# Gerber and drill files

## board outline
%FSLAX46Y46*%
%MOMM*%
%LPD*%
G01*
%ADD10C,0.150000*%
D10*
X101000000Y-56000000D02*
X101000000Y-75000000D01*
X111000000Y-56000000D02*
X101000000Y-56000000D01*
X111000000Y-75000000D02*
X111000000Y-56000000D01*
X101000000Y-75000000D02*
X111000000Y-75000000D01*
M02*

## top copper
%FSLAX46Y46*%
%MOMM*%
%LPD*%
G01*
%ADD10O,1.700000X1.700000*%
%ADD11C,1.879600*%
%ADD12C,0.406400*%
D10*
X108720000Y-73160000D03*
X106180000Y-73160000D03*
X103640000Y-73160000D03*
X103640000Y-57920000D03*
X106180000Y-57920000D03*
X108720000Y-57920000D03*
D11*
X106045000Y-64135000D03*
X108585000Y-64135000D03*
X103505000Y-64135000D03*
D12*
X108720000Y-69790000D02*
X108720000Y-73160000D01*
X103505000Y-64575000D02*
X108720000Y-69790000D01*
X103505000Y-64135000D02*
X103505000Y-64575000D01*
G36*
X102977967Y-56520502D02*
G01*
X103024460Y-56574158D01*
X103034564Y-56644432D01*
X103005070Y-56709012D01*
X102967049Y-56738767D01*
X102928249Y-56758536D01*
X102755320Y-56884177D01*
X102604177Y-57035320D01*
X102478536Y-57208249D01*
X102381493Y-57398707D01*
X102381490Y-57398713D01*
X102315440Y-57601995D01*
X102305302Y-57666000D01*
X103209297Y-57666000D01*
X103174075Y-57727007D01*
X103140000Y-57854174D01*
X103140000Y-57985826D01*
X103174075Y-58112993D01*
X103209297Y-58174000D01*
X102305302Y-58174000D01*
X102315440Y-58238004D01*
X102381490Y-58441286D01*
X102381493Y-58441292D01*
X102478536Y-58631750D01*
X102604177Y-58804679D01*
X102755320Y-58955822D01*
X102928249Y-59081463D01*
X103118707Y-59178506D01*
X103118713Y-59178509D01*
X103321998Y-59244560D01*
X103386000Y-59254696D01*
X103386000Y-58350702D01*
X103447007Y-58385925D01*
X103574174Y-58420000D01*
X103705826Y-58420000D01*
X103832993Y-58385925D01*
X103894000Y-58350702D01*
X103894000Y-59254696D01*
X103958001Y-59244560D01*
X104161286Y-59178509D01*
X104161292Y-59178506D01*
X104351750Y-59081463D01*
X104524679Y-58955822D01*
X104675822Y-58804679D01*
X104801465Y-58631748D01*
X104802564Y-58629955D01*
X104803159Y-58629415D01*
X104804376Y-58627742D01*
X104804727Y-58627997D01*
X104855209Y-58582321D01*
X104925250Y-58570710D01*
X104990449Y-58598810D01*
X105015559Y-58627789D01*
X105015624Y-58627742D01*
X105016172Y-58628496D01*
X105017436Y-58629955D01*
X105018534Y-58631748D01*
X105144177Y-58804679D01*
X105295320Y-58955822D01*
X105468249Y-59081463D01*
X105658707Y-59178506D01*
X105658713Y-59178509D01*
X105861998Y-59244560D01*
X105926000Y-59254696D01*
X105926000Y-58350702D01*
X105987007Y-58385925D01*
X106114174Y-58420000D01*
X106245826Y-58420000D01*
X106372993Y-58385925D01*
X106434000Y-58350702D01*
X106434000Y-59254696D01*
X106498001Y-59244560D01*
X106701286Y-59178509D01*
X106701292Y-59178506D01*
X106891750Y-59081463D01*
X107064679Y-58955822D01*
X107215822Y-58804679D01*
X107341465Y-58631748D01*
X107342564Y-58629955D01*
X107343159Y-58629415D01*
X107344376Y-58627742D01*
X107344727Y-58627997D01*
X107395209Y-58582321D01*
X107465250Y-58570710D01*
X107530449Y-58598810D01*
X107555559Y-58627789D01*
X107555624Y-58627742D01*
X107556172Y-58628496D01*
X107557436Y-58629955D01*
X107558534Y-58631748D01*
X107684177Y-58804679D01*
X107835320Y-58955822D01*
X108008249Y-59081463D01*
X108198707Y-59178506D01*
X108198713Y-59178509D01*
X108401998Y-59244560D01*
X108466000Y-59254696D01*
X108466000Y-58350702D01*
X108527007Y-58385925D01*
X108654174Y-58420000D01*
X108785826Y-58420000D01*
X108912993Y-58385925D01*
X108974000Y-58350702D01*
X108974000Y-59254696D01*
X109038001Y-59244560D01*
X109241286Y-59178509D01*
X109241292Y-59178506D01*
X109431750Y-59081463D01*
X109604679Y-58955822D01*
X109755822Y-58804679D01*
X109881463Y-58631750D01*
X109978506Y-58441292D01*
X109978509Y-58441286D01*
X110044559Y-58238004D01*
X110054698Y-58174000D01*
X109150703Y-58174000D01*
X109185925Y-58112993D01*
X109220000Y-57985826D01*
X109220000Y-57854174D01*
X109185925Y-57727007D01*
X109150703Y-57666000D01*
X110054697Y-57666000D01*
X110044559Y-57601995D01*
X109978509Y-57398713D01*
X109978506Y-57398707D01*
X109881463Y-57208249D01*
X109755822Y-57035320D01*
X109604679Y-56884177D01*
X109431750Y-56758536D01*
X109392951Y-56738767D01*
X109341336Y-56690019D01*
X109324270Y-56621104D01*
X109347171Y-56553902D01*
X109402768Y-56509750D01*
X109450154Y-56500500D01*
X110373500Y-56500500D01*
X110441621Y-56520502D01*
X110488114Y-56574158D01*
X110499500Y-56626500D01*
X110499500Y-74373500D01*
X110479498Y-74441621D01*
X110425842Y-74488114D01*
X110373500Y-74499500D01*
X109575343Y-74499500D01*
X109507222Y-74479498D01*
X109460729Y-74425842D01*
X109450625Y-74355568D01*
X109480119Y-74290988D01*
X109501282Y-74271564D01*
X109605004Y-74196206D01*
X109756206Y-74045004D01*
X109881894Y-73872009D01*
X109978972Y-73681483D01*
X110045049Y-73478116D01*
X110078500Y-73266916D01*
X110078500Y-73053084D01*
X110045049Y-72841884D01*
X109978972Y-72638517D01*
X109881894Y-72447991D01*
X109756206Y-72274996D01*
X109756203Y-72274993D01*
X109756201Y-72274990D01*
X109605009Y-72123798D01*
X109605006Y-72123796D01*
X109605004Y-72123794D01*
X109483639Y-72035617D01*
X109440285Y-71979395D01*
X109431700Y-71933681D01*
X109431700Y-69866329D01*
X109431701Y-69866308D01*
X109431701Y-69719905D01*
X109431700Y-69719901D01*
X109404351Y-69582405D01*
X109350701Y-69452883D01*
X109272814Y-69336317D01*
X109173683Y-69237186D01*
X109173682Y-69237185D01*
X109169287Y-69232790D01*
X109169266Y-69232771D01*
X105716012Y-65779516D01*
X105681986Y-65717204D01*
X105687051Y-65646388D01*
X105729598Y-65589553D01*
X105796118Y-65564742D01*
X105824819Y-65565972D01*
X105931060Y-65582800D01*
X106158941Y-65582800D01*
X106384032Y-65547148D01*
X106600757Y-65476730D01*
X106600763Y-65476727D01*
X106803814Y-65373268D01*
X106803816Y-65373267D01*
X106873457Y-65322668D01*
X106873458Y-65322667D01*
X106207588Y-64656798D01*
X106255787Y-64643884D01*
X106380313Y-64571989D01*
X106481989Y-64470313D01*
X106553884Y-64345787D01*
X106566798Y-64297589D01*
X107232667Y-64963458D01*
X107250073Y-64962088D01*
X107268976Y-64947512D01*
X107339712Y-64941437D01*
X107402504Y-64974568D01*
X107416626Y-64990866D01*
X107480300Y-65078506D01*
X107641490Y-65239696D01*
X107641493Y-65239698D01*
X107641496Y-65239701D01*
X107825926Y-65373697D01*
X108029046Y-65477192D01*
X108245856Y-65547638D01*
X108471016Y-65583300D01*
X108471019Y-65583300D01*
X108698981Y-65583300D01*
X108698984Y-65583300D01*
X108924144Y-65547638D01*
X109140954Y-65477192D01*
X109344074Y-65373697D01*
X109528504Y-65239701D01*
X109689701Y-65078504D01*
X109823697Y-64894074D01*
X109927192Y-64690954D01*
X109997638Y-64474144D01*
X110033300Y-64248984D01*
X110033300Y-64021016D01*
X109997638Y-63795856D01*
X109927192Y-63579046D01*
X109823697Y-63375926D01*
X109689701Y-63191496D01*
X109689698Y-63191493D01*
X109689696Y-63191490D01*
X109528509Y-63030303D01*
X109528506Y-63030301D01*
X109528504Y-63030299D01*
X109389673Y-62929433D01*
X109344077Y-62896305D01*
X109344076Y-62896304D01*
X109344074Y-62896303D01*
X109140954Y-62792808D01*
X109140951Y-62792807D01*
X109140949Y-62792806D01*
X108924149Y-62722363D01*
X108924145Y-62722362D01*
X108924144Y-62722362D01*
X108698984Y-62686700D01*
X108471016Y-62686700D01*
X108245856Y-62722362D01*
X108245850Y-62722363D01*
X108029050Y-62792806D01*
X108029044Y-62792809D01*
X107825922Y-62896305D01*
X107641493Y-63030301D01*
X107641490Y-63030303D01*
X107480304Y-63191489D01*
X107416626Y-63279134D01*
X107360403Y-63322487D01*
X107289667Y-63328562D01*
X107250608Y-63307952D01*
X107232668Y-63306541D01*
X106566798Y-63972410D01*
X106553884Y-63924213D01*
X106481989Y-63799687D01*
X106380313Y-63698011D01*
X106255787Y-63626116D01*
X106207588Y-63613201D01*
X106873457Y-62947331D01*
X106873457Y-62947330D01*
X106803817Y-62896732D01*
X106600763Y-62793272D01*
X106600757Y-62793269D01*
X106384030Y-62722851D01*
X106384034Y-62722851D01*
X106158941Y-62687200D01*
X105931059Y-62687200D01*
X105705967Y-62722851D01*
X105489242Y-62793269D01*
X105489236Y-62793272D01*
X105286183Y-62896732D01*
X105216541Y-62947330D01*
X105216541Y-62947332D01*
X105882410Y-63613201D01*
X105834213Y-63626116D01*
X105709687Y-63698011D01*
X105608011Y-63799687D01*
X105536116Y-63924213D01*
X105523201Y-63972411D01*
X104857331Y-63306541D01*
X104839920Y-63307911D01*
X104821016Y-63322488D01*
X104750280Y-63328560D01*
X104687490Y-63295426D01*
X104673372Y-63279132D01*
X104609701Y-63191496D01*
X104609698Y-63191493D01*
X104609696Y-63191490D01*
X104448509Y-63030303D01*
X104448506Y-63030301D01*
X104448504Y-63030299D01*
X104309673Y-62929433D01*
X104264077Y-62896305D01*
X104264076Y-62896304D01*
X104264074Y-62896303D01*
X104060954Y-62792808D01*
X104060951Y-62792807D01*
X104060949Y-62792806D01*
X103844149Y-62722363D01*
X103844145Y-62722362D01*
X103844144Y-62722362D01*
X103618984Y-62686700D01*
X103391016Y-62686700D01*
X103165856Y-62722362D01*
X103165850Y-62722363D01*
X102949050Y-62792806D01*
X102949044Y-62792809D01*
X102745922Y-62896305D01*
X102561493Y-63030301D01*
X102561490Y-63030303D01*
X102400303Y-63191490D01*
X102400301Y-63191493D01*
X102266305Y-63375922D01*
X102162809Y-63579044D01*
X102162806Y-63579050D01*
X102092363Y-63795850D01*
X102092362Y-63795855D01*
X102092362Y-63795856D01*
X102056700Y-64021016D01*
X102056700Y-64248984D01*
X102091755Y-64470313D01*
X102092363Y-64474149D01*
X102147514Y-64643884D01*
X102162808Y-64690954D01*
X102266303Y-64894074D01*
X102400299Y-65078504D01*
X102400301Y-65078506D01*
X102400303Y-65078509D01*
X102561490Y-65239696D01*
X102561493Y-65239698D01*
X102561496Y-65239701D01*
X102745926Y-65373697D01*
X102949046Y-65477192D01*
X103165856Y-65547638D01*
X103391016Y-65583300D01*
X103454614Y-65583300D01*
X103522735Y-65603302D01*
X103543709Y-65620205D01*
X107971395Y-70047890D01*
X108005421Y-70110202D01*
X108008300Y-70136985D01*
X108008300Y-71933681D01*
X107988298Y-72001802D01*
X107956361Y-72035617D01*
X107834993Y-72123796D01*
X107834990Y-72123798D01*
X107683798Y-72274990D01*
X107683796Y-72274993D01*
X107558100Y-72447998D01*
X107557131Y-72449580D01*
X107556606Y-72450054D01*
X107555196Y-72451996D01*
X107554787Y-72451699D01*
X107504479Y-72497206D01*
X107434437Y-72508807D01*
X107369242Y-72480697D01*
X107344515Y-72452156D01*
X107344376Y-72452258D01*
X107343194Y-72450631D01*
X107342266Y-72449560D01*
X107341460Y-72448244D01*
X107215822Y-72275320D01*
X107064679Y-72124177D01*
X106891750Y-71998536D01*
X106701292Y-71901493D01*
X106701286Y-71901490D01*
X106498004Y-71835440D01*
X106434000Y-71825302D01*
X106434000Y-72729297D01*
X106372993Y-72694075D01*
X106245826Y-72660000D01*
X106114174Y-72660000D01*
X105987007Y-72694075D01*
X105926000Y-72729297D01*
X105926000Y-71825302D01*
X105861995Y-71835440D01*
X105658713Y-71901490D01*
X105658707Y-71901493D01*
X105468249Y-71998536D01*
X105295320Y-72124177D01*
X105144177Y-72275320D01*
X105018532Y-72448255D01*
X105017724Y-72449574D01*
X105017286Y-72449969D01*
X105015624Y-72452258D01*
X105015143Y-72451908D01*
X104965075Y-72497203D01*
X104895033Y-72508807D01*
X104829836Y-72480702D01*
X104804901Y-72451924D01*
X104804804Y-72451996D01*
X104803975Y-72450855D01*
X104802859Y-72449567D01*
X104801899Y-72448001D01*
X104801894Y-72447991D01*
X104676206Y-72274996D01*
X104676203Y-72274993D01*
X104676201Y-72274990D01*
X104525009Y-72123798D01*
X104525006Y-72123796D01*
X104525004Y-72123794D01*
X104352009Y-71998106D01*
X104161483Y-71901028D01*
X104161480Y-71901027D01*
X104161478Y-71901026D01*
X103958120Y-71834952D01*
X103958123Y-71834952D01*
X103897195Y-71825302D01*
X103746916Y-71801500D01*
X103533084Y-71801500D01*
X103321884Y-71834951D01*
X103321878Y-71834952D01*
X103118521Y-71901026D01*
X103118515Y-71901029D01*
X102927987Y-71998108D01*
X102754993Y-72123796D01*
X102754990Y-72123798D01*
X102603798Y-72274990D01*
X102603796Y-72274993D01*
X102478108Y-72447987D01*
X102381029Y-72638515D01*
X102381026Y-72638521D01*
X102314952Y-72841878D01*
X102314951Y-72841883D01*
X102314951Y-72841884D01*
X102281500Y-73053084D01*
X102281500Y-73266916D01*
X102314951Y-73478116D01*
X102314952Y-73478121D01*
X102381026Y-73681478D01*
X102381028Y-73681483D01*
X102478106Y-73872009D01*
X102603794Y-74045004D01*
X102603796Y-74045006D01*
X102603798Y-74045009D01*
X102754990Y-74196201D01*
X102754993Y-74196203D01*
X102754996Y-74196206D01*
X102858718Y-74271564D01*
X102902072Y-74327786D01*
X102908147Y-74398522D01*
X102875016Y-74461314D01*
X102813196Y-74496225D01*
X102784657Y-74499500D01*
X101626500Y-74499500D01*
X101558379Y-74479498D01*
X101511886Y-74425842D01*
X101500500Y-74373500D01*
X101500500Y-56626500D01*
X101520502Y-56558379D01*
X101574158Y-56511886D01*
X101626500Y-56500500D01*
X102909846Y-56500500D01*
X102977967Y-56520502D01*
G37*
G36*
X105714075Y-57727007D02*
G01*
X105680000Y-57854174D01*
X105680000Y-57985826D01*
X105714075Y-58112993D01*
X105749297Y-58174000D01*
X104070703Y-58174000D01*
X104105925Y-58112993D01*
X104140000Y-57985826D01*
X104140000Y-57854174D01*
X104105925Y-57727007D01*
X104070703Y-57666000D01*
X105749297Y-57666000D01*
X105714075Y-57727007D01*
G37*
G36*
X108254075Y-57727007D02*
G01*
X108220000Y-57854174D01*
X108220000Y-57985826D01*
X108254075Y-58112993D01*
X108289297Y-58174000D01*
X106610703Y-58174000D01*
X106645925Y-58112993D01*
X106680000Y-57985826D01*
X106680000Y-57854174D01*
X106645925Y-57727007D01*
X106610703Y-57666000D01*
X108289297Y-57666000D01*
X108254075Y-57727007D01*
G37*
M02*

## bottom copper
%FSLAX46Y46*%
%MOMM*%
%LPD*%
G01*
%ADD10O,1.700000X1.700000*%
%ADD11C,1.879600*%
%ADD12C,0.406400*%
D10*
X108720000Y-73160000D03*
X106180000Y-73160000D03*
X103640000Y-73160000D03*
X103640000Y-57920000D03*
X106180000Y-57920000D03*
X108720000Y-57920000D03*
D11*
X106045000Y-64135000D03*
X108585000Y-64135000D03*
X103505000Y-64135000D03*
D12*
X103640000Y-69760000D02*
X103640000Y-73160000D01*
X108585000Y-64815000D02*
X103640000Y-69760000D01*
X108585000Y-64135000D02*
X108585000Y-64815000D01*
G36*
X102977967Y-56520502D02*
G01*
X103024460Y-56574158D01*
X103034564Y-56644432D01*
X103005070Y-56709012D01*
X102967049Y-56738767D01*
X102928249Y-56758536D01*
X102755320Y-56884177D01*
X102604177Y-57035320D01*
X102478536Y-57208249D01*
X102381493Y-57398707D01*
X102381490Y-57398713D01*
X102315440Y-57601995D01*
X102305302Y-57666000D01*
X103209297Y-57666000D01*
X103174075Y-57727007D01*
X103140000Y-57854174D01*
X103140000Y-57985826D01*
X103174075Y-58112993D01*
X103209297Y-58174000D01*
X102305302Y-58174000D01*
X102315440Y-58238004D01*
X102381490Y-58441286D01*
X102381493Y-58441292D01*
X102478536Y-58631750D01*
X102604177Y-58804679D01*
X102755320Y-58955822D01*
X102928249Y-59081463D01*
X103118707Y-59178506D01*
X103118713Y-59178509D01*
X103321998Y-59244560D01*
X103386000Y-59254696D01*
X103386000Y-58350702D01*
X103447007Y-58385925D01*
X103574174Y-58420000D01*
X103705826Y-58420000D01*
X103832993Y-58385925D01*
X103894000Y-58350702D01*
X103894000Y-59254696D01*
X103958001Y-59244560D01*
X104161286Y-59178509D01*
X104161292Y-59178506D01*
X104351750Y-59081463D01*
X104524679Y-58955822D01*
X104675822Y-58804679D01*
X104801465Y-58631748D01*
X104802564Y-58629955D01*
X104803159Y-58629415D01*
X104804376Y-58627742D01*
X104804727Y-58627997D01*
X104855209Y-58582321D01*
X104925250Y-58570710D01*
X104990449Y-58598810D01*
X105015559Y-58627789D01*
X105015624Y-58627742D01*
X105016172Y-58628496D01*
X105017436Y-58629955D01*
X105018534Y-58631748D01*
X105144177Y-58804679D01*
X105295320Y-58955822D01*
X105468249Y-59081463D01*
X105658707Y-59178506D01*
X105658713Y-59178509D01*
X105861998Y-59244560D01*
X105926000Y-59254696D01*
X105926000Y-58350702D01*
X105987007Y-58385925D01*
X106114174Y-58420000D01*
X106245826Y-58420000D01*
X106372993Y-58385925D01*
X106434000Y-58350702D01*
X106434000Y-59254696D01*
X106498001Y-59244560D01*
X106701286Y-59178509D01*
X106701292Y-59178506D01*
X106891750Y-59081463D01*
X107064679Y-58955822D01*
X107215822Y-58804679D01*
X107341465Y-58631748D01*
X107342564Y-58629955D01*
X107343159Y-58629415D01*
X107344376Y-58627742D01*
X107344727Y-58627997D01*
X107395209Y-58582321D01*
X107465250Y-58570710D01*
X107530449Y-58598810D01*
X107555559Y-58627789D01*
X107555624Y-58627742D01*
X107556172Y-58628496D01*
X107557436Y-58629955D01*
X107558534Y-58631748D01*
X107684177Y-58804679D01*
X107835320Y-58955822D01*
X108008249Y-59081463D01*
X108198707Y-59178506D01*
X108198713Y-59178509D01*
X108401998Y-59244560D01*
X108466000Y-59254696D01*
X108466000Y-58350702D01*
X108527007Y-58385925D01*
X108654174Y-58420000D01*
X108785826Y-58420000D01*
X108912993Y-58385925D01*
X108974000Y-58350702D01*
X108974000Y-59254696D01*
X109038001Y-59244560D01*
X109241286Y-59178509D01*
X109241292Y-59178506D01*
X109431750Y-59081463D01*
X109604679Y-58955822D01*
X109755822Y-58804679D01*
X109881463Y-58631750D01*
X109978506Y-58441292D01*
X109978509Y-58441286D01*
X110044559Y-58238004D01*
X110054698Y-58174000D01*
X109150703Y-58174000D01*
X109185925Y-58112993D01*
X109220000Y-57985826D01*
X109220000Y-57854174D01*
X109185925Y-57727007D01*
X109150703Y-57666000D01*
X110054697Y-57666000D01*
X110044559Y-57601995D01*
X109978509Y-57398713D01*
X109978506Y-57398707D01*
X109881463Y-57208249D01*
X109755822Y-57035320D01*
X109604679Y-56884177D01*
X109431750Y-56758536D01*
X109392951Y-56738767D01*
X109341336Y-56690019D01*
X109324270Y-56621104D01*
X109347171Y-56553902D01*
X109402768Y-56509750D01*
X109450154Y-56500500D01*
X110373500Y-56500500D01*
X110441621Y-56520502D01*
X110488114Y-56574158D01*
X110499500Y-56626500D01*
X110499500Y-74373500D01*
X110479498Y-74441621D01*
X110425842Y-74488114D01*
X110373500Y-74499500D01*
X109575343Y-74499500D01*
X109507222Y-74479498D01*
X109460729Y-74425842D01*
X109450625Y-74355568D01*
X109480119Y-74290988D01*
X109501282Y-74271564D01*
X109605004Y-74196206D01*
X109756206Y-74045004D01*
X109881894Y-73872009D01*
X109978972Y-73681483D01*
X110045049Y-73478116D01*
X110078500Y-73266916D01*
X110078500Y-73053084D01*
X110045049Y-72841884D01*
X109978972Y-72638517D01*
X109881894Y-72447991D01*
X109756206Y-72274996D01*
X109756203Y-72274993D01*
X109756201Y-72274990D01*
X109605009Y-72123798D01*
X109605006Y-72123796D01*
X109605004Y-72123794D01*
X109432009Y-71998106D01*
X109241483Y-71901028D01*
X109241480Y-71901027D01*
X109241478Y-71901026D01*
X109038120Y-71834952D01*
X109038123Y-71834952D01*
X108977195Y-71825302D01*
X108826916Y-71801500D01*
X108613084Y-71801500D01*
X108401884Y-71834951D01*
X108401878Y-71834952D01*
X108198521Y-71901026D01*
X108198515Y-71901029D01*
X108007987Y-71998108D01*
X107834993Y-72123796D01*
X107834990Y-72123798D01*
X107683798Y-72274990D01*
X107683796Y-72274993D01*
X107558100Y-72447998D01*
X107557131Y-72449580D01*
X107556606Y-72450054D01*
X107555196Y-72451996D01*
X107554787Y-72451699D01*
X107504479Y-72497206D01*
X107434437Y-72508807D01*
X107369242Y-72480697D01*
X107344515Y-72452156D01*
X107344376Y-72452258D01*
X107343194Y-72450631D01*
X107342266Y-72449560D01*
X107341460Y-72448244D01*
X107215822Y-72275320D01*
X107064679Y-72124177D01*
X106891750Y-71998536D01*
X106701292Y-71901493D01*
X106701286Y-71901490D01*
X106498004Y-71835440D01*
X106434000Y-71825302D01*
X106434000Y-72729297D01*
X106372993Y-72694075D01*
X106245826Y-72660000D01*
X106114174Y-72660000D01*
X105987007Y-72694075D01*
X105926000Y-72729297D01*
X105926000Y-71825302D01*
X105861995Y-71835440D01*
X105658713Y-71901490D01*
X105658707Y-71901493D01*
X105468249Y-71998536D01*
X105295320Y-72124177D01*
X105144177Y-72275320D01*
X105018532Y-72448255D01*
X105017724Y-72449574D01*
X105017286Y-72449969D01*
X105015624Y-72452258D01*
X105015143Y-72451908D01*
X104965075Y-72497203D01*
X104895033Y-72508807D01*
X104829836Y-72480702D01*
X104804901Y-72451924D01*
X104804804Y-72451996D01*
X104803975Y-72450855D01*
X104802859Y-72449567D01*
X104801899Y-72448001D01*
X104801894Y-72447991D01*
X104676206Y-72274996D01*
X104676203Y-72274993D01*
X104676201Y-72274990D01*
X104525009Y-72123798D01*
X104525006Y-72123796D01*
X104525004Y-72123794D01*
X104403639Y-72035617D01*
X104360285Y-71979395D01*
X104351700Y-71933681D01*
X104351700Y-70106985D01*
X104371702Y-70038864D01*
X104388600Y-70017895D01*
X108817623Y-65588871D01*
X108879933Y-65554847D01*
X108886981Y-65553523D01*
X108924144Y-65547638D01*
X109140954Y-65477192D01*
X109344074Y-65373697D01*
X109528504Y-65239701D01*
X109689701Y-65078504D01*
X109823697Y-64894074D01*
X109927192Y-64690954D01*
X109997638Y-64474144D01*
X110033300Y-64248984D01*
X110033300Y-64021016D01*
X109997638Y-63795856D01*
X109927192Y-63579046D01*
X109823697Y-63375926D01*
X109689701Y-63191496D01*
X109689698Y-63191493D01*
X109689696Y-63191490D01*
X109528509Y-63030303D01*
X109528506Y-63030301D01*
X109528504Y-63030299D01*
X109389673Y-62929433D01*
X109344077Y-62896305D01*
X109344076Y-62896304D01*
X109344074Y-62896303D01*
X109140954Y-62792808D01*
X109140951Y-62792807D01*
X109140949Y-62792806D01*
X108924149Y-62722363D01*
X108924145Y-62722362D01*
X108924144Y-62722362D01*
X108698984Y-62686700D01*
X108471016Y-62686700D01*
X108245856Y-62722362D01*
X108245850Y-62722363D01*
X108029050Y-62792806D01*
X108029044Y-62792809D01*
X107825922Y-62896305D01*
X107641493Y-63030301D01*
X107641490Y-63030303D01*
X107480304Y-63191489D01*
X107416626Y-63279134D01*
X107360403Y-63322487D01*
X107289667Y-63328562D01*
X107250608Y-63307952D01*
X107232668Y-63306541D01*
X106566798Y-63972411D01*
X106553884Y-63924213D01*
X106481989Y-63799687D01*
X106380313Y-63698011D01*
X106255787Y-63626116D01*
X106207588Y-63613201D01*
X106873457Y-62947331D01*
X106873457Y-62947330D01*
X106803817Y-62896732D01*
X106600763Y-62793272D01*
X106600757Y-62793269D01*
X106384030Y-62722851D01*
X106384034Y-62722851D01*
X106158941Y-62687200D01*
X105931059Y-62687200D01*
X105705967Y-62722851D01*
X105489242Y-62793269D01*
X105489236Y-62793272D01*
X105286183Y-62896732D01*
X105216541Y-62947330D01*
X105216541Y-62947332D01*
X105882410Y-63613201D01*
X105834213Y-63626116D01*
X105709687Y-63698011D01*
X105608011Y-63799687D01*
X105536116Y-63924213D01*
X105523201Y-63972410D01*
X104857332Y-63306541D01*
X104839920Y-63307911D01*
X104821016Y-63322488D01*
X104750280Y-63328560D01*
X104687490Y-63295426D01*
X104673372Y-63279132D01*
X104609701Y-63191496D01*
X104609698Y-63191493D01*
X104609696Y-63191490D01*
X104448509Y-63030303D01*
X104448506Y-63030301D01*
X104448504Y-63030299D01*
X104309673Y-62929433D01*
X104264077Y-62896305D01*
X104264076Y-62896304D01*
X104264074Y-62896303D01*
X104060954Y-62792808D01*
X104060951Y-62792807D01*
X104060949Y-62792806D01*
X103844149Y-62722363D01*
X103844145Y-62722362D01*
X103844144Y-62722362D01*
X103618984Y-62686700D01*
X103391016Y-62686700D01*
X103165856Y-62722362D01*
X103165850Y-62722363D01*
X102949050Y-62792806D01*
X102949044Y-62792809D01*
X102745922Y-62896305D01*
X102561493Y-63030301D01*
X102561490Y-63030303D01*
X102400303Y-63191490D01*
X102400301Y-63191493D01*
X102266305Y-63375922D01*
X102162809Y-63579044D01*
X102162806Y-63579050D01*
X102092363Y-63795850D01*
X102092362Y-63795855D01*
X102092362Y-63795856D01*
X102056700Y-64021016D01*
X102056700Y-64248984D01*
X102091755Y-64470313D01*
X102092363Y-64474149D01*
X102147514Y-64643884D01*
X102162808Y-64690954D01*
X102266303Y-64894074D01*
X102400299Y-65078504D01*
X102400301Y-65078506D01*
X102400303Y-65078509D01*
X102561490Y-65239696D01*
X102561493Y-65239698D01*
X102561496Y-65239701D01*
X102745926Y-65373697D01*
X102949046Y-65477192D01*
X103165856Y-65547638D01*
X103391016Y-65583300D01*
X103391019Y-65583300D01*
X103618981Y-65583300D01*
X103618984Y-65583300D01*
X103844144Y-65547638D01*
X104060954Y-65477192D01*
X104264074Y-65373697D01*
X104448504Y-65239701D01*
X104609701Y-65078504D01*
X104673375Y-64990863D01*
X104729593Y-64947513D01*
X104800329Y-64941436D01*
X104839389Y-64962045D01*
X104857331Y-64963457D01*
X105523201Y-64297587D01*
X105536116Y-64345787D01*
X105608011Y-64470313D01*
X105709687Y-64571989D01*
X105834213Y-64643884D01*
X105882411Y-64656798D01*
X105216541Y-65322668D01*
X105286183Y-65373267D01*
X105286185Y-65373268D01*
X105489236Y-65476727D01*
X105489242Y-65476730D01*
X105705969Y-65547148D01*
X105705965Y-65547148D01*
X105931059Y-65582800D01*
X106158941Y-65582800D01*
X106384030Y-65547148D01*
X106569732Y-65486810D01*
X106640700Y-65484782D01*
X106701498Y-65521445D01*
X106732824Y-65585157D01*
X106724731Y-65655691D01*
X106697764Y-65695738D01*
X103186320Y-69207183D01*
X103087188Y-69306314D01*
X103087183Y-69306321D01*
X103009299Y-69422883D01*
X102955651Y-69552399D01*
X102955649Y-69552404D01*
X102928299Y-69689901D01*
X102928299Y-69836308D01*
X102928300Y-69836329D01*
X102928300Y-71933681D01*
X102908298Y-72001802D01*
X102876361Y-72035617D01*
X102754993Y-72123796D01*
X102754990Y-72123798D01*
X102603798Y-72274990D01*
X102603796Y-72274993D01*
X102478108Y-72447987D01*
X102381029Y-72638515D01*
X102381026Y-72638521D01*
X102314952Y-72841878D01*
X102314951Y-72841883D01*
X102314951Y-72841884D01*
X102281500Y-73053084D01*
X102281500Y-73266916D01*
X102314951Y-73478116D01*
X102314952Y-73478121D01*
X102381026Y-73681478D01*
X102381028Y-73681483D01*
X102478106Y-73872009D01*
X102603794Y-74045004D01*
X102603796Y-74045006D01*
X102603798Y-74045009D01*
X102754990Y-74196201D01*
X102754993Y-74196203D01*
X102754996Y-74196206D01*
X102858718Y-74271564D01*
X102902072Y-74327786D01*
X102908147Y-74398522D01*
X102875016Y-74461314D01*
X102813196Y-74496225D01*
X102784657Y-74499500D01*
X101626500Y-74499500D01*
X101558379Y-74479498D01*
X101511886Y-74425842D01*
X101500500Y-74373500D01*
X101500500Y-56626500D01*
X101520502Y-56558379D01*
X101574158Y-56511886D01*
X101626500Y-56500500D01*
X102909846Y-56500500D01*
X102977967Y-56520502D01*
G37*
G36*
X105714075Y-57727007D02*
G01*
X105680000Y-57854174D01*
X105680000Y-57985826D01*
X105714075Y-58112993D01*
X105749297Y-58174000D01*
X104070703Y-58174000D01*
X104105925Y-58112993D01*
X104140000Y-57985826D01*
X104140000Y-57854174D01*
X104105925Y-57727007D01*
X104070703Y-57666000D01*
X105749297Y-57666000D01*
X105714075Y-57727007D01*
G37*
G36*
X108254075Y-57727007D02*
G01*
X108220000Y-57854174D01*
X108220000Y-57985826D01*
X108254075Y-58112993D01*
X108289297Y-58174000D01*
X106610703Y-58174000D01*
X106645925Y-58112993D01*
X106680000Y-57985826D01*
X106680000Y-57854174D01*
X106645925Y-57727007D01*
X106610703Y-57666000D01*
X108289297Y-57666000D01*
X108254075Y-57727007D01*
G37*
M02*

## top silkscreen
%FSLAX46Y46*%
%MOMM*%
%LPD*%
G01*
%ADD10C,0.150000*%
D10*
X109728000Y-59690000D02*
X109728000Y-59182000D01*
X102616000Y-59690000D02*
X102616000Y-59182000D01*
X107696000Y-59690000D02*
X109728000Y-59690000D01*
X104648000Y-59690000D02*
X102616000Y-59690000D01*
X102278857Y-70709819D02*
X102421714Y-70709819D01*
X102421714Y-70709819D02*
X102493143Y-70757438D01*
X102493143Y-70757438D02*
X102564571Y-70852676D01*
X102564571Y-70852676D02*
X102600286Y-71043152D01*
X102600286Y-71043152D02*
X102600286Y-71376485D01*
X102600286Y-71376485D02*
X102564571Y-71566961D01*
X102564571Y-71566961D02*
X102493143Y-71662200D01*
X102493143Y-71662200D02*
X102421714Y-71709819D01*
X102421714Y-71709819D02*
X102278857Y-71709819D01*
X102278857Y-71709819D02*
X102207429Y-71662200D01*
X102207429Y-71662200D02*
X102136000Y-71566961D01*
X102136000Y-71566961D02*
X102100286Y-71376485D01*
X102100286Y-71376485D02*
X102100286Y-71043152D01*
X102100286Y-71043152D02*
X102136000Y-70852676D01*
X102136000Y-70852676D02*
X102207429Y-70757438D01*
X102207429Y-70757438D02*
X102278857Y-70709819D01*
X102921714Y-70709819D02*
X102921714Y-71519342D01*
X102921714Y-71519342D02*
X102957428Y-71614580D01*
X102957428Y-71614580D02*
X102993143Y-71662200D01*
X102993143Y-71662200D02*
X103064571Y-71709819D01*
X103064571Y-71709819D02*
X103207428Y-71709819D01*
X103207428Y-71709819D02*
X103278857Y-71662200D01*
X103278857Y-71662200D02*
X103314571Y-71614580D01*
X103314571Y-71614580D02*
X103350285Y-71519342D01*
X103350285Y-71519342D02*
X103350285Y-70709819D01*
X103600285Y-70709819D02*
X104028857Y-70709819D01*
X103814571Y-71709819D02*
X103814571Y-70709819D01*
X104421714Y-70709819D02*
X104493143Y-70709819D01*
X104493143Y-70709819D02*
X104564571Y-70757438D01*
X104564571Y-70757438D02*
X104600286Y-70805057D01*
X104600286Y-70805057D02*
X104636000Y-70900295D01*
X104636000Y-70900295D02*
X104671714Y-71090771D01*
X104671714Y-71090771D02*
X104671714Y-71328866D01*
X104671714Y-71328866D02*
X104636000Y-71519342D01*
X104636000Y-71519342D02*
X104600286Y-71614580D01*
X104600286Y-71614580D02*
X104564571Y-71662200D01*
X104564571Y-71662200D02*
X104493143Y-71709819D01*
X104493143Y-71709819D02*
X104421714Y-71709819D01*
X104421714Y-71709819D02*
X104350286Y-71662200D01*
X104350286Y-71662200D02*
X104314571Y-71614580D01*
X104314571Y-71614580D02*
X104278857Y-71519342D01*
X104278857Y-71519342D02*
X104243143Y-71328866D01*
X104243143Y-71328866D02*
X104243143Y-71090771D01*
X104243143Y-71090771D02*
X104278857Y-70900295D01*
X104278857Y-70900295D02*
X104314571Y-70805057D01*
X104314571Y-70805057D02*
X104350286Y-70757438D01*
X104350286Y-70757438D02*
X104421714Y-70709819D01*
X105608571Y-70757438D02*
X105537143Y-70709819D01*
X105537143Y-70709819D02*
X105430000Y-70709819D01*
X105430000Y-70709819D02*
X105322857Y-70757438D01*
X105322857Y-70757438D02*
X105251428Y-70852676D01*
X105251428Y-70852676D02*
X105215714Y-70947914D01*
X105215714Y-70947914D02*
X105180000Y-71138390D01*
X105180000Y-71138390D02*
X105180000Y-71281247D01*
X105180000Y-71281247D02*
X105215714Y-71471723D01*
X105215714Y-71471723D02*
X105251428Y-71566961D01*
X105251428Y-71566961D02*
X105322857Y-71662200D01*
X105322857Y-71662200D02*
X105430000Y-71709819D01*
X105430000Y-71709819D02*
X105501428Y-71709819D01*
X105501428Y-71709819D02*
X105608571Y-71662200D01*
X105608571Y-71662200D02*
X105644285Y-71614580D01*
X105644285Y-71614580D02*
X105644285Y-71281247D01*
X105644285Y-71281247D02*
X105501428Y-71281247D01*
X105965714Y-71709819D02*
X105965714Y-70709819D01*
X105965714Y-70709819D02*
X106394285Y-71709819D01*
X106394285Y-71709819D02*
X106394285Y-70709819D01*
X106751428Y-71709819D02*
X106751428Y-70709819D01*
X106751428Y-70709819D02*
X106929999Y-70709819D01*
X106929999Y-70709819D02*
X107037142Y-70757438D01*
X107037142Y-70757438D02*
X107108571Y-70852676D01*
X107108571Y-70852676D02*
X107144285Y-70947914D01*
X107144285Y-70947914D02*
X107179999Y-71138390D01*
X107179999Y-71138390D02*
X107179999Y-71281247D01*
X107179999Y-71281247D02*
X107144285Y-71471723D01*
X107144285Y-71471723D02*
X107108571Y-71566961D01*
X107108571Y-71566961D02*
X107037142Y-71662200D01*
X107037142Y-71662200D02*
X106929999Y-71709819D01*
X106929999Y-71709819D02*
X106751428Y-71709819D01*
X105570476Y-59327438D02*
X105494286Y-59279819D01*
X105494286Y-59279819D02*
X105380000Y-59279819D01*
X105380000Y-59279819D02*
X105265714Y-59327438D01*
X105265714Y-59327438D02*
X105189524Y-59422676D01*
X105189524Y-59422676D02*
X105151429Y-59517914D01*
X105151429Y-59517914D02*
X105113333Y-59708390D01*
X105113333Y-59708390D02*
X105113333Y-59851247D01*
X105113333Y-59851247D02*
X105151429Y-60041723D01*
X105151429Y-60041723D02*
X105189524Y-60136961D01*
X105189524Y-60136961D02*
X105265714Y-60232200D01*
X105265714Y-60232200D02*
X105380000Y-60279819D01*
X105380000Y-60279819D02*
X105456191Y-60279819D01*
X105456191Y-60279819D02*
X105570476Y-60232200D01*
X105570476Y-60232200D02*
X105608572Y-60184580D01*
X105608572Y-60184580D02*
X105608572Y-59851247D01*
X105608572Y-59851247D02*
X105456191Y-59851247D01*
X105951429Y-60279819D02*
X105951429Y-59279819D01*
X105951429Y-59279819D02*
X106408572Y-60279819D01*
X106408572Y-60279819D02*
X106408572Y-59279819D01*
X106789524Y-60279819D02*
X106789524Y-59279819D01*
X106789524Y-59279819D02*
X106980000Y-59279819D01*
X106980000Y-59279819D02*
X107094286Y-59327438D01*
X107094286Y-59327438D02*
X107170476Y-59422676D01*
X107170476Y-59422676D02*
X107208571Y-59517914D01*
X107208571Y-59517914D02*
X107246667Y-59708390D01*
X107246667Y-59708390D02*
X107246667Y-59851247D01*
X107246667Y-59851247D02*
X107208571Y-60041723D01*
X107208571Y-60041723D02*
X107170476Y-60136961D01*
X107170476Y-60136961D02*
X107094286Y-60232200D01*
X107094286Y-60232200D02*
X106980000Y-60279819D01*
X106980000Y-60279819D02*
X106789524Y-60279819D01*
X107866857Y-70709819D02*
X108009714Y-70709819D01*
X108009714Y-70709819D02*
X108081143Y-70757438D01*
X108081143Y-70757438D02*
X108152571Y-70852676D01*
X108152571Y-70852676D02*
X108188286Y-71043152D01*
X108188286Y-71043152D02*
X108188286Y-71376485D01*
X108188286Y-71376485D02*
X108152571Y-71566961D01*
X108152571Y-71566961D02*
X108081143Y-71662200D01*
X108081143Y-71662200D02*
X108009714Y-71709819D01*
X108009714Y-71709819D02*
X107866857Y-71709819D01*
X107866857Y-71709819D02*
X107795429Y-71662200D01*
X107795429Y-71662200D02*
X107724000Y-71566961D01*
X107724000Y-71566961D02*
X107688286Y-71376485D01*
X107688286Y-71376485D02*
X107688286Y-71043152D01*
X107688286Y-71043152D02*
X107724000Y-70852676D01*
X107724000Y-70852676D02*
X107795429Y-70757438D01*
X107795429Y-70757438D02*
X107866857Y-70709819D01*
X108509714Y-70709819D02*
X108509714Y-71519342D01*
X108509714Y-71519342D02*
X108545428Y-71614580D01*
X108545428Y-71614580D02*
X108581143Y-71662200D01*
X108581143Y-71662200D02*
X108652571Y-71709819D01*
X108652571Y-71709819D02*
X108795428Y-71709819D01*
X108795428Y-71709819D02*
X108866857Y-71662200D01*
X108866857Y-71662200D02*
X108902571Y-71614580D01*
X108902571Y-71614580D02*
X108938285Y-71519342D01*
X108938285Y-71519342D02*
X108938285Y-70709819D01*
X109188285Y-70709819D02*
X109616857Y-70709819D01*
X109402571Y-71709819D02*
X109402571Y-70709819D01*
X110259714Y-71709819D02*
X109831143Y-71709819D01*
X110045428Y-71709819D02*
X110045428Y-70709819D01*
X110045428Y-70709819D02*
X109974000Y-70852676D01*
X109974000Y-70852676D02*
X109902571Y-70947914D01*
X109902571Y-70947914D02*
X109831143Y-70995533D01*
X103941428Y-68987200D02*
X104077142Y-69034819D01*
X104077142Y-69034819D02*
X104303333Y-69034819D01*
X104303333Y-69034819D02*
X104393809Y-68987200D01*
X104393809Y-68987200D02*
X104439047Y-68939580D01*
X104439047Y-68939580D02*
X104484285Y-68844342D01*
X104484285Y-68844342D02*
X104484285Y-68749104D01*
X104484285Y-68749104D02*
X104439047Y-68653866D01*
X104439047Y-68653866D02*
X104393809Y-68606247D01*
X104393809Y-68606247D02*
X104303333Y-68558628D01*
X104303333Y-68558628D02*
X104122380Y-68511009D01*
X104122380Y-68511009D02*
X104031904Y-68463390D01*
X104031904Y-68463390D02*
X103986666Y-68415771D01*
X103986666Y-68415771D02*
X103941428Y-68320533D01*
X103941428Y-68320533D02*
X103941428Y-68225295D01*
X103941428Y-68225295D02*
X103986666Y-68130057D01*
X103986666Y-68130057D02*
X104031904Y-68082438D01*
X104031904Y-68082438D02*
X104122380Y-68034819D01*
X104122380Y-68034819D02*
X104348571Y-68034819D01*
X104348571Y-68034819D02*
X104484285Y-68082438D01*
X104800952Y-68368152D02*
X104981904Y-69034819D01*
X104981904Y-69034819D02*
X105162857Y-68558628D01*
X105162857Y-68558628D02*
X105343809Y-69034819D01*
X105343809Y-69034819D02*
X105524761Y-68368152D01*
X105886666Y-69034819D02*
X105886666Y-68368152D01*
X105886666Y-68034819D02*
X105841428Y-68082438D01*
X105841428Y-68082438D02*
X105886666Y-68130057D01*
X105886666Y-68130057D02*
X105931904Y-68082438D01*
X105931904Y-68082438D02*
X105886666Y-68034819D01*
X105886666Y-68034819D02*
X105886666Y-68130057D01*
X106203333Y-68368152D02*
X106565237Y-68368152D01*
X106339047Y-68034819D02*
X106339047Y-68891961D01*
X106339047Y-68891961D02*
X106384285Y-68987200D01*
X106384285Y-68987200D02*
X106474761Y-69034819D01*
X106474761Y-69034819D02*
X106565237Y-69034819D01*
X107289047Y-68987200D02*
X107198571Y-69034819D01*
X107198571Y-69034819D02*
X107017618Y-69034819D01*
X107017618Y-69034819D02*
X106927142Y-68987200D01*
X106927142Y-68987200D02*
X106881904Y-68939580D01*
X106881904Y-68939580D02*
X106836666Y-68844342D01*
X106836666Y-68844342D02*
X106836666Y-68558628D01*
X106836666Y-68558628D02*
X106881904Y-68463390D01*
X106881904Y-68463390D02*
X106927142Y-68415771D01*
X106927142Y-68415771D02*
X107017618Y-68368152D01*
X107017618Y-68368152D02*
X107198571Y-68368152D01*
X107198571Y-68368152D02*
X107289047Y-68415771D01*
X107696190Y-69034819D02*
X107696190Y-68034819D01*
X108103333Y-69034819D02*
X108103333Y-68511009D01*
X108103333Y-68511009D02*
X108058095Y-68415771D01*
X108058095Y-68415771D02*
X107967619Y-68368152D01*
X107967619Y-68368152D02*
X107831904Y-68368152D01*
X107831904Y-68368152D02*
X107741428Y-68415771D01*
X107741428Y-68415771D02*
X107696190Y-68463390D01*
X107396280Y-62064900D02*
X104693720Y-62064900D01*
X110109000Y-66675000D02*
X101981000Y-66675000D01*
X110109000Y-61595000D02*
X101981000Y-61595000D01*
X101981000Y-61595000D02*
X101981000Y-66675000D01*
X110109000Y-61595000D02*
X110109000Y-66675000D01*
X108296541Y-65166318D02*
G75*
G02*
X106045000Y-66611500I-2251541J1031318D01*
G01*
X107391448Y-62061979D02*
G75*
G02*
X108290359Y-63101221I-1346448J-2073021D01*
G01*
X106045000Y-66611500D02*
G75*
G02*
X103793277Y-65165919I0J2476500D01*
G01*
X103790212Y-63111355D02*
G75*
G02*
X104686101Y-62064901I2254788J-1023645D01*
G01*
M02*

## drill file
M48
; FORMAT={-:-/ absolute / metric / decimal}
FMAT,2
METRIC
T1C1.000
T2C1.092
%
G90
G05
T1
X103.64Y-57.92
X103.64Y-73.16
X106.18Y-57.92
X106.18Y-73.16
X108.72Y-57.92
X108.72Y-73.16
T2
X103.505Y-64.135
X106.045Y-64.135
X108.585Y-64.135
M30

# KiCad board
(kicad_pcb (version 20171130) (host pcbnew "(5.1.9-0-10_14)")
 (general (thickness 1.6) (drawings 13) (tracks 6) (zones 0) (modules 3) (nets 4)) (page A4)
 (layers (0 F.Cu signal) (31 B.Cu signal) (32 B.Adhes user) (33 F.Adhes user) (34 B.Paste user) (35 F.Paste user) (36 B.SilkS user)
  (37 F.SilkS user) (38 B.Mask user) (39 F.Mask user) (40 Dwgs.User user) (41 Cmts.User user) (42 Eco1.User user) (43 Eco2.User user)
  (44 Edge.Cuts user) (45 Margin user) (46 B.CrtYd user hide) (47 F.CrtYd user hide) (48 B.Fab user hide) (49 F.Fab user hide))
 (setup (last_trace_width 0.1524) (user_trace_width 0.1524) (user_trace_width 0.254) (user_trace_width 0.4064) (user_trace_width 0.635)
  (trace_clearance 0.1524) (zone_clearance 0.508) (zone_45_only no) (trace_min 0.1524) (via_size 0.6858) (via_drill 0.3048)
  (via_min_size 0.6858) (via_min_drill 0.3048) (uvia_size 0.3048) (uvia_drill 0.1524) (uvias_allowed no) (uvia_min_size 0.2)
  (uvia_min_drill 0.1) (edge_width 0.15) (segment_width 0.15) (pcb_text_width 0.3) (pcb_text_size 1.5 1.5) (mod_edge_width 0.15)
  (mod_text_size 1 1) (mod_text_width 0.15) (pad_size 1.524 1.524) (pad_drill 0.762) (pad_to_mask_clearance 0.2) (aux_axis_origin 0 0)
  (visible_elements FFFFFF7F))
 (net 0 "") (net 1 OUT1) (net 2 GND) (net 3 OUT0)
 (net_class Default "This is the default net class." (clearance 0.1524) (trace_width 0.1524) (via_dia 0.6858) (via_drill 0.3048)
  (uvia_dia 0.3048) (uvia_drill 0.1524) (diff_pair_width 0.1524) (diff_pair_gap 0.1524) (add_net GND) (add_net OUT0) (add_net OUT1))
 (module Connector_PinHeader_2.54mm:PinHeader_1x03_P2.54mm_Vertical (layer B.Cu) (at 103.64 73.16 270)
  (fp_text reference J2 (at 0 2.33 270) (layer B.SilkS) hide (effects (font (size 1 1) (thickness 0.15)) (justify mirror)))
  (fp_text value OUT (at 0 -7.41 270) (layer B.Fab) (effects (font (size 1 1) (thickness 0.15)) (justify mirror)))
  (pad 3 thru_hole oval (at 0 -5.08 270) (size 1.7 1.7) (drill 1) (layers *.Cu *.Mask) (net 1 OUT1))
  (pad 2 thru_hole oval (at 0 -2.54 270) (size 1.7 1.7) (drill 1) (layers *.Cu *.Mask) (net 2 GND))
  (pad 1 thru_hole oval (at 0 0 270) (size 1.7 1.7) (drill 1) (layers *.Cu *.Mask) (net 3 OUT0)))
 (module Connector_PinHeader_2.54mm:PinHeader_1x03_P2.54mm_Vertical (layer B.Cu) (at 103.64 57.92 270)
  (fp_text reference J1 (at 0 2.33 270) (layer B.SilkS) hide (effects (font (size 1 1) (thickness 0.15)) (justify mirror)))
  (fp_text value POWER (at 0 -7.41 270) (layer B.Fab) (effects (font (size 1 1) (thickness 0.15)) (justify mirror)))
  (pad 1 thru_hole oval (at 0 0 270) (size 1.7 1.7) (drill 1) (layers *.Cu *.Mask) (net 2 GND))
  (pad 2 thru_hole oval (at 0 -2.54 270) (size 1.7 1.7) (drill 1) (layers *.Cu *.Mask) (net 2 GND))
  (pad 3 thru_hole oval (at 0 -5.08 270) (size 1.7 1.7) (drill 1) (layers *.Cu *.Mask) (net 2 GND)))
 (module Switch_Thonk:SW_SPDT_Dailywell (layer F.Cu) (at 106.045 64.135 270)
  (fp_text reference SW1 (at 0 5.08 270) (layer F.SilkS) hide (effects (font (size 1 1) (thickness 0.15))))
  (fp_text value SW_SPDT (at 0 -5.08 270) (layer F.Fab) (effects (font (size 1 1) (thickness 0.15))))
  (fp_line (start -2.0701 -1.35128) (end -2.0701 1.35128) (layer F.SilkS) (width 0.15))
  (fp_line (start 2.54 -4.064) (end 2.54 4.064) (layer F.SilkS) (width 0.15))
  (fp_line (start -2.54 -4.064) (end -2.54 4.064) (layer F.SilkS) (width 0.15))
  (fp_line (start -2.54 4.064) (end 2.54 4.064) (layer F.SilkS) (width 0.15))
  (fp_line (start -2.54 -4.064) (end 2.54 -4.064) (layer F.SilkS) (width 0.15))
  (fp_arc (start 0 0) (end 2.4765 0) (angle -65.38985762) (layer F.SilkS) (width 0.15))
  (fp_arc (start 0 0) (end -1.033779 -2.245359) (angle -32.27419574) (layer F.SilkS) (width 0.15))
  (fp_arc (start 0 0) (end 2.4765 0) (angle 65.4) (layer F.SilkS) (width 0.15))
  (fp_arc (start 0 0) (end -2.070099 1.358899) (angle -32.3) (layer F.SilkS) (width 0.15))
  (pad 2 thru_hole circle (at 0 0 270) (size 1.8796 1.8796) (drill 1.0922) (layers *.Cu *.Mask) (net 2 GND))
  (pad 3 thru_hole circle (at 0 -2.54 270) (size 1.8796 1.8796) (drill 1.0922) (layers *.Cu *.Mask) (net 3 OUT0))
  (pad 1 thru_hole circle (at 0 2.54 270) (size 1.8796 1.8796) (drill 1.0922) (layers *.Cu *.Mask) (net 1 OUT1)))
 (gr_line (start 109.728 59.69) (end 109.728 59.182) (layer F.SilkS) (width 0.15))
 (gr_line (start 102.616 59.69) (end 102.616 59.182) (layer F.SilkS) (width 0.15))
 (gr_line (start 107.696 59.69) (end 109.728 59.69) (layer F.SilkS) (width 0.15))
 (gr_line (start 104.648 59.69) (end 102.616 59.69) (layer F.SilkS) (width 0.15))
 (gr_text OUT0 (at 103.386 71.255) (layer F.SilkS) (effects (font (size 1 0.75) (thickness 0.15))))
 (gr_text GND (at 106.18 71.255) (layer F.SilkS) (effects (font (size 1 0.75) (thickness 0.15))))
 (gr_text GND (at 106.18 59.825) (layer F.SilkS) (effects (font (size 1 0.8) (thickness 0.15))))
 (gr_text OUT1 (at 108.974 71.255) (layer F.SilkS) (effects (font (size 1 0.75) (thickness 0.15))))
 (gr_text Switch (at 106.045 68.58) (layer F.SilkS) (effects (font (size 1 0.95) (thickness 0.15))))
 (gr_line (start 101 56) (end 101 75) (layer Edge.Cuts) (width 0.15))
 (gr_line (start 111 56) (end 101 56) (layer Edge.Cuts) (width 0.15))
 (gr_line (start 111 75) (end 111 56) (layer Edge.Cuts) (width 0.15))
 (gr_line (start 101 75) (end 111 75) (layer Edge.Cuts) (width 0.15))
 (segment (start 108.72 69.79) (end 108.72 73.16) (width 0.4064) (layer F.Cu) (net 1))
 (segment (start 103.505 64.575) (end 108.72 69.79) (width 0.4064) (layer F.Cu) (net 1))
 (segment (start 103.505 64.135) (end 103.505 64.575) (width 0.4064) (layer F.Cu) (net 1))
 (segment (start 103.64 69.76) (end 103.64 73.16) (width 0.4064) (layer B.Cu) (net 3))
 (segment (start 108.585 64.815) (end 103.64 69.76) (width 0.4064) (layer B.Cu) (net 3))
 (segment (start 108.585 64.135) (end 108.585 64.815) (width 0.4064) (layer B.Cu) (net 3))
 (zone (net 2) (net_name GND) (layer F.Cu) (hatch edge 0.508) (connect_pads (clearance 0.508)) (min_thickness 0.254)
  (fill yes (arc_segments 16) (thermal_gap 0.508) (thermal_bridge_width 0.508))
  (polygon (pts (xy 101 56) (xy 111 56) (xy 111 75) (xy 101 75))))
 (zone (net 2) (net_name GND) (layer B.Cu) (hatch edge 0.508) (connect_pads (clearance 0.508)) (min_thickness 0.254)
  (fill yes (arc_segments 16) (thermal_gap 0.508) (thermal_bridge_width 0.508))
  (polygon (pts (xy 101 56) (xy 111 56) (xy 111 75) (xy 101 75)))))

